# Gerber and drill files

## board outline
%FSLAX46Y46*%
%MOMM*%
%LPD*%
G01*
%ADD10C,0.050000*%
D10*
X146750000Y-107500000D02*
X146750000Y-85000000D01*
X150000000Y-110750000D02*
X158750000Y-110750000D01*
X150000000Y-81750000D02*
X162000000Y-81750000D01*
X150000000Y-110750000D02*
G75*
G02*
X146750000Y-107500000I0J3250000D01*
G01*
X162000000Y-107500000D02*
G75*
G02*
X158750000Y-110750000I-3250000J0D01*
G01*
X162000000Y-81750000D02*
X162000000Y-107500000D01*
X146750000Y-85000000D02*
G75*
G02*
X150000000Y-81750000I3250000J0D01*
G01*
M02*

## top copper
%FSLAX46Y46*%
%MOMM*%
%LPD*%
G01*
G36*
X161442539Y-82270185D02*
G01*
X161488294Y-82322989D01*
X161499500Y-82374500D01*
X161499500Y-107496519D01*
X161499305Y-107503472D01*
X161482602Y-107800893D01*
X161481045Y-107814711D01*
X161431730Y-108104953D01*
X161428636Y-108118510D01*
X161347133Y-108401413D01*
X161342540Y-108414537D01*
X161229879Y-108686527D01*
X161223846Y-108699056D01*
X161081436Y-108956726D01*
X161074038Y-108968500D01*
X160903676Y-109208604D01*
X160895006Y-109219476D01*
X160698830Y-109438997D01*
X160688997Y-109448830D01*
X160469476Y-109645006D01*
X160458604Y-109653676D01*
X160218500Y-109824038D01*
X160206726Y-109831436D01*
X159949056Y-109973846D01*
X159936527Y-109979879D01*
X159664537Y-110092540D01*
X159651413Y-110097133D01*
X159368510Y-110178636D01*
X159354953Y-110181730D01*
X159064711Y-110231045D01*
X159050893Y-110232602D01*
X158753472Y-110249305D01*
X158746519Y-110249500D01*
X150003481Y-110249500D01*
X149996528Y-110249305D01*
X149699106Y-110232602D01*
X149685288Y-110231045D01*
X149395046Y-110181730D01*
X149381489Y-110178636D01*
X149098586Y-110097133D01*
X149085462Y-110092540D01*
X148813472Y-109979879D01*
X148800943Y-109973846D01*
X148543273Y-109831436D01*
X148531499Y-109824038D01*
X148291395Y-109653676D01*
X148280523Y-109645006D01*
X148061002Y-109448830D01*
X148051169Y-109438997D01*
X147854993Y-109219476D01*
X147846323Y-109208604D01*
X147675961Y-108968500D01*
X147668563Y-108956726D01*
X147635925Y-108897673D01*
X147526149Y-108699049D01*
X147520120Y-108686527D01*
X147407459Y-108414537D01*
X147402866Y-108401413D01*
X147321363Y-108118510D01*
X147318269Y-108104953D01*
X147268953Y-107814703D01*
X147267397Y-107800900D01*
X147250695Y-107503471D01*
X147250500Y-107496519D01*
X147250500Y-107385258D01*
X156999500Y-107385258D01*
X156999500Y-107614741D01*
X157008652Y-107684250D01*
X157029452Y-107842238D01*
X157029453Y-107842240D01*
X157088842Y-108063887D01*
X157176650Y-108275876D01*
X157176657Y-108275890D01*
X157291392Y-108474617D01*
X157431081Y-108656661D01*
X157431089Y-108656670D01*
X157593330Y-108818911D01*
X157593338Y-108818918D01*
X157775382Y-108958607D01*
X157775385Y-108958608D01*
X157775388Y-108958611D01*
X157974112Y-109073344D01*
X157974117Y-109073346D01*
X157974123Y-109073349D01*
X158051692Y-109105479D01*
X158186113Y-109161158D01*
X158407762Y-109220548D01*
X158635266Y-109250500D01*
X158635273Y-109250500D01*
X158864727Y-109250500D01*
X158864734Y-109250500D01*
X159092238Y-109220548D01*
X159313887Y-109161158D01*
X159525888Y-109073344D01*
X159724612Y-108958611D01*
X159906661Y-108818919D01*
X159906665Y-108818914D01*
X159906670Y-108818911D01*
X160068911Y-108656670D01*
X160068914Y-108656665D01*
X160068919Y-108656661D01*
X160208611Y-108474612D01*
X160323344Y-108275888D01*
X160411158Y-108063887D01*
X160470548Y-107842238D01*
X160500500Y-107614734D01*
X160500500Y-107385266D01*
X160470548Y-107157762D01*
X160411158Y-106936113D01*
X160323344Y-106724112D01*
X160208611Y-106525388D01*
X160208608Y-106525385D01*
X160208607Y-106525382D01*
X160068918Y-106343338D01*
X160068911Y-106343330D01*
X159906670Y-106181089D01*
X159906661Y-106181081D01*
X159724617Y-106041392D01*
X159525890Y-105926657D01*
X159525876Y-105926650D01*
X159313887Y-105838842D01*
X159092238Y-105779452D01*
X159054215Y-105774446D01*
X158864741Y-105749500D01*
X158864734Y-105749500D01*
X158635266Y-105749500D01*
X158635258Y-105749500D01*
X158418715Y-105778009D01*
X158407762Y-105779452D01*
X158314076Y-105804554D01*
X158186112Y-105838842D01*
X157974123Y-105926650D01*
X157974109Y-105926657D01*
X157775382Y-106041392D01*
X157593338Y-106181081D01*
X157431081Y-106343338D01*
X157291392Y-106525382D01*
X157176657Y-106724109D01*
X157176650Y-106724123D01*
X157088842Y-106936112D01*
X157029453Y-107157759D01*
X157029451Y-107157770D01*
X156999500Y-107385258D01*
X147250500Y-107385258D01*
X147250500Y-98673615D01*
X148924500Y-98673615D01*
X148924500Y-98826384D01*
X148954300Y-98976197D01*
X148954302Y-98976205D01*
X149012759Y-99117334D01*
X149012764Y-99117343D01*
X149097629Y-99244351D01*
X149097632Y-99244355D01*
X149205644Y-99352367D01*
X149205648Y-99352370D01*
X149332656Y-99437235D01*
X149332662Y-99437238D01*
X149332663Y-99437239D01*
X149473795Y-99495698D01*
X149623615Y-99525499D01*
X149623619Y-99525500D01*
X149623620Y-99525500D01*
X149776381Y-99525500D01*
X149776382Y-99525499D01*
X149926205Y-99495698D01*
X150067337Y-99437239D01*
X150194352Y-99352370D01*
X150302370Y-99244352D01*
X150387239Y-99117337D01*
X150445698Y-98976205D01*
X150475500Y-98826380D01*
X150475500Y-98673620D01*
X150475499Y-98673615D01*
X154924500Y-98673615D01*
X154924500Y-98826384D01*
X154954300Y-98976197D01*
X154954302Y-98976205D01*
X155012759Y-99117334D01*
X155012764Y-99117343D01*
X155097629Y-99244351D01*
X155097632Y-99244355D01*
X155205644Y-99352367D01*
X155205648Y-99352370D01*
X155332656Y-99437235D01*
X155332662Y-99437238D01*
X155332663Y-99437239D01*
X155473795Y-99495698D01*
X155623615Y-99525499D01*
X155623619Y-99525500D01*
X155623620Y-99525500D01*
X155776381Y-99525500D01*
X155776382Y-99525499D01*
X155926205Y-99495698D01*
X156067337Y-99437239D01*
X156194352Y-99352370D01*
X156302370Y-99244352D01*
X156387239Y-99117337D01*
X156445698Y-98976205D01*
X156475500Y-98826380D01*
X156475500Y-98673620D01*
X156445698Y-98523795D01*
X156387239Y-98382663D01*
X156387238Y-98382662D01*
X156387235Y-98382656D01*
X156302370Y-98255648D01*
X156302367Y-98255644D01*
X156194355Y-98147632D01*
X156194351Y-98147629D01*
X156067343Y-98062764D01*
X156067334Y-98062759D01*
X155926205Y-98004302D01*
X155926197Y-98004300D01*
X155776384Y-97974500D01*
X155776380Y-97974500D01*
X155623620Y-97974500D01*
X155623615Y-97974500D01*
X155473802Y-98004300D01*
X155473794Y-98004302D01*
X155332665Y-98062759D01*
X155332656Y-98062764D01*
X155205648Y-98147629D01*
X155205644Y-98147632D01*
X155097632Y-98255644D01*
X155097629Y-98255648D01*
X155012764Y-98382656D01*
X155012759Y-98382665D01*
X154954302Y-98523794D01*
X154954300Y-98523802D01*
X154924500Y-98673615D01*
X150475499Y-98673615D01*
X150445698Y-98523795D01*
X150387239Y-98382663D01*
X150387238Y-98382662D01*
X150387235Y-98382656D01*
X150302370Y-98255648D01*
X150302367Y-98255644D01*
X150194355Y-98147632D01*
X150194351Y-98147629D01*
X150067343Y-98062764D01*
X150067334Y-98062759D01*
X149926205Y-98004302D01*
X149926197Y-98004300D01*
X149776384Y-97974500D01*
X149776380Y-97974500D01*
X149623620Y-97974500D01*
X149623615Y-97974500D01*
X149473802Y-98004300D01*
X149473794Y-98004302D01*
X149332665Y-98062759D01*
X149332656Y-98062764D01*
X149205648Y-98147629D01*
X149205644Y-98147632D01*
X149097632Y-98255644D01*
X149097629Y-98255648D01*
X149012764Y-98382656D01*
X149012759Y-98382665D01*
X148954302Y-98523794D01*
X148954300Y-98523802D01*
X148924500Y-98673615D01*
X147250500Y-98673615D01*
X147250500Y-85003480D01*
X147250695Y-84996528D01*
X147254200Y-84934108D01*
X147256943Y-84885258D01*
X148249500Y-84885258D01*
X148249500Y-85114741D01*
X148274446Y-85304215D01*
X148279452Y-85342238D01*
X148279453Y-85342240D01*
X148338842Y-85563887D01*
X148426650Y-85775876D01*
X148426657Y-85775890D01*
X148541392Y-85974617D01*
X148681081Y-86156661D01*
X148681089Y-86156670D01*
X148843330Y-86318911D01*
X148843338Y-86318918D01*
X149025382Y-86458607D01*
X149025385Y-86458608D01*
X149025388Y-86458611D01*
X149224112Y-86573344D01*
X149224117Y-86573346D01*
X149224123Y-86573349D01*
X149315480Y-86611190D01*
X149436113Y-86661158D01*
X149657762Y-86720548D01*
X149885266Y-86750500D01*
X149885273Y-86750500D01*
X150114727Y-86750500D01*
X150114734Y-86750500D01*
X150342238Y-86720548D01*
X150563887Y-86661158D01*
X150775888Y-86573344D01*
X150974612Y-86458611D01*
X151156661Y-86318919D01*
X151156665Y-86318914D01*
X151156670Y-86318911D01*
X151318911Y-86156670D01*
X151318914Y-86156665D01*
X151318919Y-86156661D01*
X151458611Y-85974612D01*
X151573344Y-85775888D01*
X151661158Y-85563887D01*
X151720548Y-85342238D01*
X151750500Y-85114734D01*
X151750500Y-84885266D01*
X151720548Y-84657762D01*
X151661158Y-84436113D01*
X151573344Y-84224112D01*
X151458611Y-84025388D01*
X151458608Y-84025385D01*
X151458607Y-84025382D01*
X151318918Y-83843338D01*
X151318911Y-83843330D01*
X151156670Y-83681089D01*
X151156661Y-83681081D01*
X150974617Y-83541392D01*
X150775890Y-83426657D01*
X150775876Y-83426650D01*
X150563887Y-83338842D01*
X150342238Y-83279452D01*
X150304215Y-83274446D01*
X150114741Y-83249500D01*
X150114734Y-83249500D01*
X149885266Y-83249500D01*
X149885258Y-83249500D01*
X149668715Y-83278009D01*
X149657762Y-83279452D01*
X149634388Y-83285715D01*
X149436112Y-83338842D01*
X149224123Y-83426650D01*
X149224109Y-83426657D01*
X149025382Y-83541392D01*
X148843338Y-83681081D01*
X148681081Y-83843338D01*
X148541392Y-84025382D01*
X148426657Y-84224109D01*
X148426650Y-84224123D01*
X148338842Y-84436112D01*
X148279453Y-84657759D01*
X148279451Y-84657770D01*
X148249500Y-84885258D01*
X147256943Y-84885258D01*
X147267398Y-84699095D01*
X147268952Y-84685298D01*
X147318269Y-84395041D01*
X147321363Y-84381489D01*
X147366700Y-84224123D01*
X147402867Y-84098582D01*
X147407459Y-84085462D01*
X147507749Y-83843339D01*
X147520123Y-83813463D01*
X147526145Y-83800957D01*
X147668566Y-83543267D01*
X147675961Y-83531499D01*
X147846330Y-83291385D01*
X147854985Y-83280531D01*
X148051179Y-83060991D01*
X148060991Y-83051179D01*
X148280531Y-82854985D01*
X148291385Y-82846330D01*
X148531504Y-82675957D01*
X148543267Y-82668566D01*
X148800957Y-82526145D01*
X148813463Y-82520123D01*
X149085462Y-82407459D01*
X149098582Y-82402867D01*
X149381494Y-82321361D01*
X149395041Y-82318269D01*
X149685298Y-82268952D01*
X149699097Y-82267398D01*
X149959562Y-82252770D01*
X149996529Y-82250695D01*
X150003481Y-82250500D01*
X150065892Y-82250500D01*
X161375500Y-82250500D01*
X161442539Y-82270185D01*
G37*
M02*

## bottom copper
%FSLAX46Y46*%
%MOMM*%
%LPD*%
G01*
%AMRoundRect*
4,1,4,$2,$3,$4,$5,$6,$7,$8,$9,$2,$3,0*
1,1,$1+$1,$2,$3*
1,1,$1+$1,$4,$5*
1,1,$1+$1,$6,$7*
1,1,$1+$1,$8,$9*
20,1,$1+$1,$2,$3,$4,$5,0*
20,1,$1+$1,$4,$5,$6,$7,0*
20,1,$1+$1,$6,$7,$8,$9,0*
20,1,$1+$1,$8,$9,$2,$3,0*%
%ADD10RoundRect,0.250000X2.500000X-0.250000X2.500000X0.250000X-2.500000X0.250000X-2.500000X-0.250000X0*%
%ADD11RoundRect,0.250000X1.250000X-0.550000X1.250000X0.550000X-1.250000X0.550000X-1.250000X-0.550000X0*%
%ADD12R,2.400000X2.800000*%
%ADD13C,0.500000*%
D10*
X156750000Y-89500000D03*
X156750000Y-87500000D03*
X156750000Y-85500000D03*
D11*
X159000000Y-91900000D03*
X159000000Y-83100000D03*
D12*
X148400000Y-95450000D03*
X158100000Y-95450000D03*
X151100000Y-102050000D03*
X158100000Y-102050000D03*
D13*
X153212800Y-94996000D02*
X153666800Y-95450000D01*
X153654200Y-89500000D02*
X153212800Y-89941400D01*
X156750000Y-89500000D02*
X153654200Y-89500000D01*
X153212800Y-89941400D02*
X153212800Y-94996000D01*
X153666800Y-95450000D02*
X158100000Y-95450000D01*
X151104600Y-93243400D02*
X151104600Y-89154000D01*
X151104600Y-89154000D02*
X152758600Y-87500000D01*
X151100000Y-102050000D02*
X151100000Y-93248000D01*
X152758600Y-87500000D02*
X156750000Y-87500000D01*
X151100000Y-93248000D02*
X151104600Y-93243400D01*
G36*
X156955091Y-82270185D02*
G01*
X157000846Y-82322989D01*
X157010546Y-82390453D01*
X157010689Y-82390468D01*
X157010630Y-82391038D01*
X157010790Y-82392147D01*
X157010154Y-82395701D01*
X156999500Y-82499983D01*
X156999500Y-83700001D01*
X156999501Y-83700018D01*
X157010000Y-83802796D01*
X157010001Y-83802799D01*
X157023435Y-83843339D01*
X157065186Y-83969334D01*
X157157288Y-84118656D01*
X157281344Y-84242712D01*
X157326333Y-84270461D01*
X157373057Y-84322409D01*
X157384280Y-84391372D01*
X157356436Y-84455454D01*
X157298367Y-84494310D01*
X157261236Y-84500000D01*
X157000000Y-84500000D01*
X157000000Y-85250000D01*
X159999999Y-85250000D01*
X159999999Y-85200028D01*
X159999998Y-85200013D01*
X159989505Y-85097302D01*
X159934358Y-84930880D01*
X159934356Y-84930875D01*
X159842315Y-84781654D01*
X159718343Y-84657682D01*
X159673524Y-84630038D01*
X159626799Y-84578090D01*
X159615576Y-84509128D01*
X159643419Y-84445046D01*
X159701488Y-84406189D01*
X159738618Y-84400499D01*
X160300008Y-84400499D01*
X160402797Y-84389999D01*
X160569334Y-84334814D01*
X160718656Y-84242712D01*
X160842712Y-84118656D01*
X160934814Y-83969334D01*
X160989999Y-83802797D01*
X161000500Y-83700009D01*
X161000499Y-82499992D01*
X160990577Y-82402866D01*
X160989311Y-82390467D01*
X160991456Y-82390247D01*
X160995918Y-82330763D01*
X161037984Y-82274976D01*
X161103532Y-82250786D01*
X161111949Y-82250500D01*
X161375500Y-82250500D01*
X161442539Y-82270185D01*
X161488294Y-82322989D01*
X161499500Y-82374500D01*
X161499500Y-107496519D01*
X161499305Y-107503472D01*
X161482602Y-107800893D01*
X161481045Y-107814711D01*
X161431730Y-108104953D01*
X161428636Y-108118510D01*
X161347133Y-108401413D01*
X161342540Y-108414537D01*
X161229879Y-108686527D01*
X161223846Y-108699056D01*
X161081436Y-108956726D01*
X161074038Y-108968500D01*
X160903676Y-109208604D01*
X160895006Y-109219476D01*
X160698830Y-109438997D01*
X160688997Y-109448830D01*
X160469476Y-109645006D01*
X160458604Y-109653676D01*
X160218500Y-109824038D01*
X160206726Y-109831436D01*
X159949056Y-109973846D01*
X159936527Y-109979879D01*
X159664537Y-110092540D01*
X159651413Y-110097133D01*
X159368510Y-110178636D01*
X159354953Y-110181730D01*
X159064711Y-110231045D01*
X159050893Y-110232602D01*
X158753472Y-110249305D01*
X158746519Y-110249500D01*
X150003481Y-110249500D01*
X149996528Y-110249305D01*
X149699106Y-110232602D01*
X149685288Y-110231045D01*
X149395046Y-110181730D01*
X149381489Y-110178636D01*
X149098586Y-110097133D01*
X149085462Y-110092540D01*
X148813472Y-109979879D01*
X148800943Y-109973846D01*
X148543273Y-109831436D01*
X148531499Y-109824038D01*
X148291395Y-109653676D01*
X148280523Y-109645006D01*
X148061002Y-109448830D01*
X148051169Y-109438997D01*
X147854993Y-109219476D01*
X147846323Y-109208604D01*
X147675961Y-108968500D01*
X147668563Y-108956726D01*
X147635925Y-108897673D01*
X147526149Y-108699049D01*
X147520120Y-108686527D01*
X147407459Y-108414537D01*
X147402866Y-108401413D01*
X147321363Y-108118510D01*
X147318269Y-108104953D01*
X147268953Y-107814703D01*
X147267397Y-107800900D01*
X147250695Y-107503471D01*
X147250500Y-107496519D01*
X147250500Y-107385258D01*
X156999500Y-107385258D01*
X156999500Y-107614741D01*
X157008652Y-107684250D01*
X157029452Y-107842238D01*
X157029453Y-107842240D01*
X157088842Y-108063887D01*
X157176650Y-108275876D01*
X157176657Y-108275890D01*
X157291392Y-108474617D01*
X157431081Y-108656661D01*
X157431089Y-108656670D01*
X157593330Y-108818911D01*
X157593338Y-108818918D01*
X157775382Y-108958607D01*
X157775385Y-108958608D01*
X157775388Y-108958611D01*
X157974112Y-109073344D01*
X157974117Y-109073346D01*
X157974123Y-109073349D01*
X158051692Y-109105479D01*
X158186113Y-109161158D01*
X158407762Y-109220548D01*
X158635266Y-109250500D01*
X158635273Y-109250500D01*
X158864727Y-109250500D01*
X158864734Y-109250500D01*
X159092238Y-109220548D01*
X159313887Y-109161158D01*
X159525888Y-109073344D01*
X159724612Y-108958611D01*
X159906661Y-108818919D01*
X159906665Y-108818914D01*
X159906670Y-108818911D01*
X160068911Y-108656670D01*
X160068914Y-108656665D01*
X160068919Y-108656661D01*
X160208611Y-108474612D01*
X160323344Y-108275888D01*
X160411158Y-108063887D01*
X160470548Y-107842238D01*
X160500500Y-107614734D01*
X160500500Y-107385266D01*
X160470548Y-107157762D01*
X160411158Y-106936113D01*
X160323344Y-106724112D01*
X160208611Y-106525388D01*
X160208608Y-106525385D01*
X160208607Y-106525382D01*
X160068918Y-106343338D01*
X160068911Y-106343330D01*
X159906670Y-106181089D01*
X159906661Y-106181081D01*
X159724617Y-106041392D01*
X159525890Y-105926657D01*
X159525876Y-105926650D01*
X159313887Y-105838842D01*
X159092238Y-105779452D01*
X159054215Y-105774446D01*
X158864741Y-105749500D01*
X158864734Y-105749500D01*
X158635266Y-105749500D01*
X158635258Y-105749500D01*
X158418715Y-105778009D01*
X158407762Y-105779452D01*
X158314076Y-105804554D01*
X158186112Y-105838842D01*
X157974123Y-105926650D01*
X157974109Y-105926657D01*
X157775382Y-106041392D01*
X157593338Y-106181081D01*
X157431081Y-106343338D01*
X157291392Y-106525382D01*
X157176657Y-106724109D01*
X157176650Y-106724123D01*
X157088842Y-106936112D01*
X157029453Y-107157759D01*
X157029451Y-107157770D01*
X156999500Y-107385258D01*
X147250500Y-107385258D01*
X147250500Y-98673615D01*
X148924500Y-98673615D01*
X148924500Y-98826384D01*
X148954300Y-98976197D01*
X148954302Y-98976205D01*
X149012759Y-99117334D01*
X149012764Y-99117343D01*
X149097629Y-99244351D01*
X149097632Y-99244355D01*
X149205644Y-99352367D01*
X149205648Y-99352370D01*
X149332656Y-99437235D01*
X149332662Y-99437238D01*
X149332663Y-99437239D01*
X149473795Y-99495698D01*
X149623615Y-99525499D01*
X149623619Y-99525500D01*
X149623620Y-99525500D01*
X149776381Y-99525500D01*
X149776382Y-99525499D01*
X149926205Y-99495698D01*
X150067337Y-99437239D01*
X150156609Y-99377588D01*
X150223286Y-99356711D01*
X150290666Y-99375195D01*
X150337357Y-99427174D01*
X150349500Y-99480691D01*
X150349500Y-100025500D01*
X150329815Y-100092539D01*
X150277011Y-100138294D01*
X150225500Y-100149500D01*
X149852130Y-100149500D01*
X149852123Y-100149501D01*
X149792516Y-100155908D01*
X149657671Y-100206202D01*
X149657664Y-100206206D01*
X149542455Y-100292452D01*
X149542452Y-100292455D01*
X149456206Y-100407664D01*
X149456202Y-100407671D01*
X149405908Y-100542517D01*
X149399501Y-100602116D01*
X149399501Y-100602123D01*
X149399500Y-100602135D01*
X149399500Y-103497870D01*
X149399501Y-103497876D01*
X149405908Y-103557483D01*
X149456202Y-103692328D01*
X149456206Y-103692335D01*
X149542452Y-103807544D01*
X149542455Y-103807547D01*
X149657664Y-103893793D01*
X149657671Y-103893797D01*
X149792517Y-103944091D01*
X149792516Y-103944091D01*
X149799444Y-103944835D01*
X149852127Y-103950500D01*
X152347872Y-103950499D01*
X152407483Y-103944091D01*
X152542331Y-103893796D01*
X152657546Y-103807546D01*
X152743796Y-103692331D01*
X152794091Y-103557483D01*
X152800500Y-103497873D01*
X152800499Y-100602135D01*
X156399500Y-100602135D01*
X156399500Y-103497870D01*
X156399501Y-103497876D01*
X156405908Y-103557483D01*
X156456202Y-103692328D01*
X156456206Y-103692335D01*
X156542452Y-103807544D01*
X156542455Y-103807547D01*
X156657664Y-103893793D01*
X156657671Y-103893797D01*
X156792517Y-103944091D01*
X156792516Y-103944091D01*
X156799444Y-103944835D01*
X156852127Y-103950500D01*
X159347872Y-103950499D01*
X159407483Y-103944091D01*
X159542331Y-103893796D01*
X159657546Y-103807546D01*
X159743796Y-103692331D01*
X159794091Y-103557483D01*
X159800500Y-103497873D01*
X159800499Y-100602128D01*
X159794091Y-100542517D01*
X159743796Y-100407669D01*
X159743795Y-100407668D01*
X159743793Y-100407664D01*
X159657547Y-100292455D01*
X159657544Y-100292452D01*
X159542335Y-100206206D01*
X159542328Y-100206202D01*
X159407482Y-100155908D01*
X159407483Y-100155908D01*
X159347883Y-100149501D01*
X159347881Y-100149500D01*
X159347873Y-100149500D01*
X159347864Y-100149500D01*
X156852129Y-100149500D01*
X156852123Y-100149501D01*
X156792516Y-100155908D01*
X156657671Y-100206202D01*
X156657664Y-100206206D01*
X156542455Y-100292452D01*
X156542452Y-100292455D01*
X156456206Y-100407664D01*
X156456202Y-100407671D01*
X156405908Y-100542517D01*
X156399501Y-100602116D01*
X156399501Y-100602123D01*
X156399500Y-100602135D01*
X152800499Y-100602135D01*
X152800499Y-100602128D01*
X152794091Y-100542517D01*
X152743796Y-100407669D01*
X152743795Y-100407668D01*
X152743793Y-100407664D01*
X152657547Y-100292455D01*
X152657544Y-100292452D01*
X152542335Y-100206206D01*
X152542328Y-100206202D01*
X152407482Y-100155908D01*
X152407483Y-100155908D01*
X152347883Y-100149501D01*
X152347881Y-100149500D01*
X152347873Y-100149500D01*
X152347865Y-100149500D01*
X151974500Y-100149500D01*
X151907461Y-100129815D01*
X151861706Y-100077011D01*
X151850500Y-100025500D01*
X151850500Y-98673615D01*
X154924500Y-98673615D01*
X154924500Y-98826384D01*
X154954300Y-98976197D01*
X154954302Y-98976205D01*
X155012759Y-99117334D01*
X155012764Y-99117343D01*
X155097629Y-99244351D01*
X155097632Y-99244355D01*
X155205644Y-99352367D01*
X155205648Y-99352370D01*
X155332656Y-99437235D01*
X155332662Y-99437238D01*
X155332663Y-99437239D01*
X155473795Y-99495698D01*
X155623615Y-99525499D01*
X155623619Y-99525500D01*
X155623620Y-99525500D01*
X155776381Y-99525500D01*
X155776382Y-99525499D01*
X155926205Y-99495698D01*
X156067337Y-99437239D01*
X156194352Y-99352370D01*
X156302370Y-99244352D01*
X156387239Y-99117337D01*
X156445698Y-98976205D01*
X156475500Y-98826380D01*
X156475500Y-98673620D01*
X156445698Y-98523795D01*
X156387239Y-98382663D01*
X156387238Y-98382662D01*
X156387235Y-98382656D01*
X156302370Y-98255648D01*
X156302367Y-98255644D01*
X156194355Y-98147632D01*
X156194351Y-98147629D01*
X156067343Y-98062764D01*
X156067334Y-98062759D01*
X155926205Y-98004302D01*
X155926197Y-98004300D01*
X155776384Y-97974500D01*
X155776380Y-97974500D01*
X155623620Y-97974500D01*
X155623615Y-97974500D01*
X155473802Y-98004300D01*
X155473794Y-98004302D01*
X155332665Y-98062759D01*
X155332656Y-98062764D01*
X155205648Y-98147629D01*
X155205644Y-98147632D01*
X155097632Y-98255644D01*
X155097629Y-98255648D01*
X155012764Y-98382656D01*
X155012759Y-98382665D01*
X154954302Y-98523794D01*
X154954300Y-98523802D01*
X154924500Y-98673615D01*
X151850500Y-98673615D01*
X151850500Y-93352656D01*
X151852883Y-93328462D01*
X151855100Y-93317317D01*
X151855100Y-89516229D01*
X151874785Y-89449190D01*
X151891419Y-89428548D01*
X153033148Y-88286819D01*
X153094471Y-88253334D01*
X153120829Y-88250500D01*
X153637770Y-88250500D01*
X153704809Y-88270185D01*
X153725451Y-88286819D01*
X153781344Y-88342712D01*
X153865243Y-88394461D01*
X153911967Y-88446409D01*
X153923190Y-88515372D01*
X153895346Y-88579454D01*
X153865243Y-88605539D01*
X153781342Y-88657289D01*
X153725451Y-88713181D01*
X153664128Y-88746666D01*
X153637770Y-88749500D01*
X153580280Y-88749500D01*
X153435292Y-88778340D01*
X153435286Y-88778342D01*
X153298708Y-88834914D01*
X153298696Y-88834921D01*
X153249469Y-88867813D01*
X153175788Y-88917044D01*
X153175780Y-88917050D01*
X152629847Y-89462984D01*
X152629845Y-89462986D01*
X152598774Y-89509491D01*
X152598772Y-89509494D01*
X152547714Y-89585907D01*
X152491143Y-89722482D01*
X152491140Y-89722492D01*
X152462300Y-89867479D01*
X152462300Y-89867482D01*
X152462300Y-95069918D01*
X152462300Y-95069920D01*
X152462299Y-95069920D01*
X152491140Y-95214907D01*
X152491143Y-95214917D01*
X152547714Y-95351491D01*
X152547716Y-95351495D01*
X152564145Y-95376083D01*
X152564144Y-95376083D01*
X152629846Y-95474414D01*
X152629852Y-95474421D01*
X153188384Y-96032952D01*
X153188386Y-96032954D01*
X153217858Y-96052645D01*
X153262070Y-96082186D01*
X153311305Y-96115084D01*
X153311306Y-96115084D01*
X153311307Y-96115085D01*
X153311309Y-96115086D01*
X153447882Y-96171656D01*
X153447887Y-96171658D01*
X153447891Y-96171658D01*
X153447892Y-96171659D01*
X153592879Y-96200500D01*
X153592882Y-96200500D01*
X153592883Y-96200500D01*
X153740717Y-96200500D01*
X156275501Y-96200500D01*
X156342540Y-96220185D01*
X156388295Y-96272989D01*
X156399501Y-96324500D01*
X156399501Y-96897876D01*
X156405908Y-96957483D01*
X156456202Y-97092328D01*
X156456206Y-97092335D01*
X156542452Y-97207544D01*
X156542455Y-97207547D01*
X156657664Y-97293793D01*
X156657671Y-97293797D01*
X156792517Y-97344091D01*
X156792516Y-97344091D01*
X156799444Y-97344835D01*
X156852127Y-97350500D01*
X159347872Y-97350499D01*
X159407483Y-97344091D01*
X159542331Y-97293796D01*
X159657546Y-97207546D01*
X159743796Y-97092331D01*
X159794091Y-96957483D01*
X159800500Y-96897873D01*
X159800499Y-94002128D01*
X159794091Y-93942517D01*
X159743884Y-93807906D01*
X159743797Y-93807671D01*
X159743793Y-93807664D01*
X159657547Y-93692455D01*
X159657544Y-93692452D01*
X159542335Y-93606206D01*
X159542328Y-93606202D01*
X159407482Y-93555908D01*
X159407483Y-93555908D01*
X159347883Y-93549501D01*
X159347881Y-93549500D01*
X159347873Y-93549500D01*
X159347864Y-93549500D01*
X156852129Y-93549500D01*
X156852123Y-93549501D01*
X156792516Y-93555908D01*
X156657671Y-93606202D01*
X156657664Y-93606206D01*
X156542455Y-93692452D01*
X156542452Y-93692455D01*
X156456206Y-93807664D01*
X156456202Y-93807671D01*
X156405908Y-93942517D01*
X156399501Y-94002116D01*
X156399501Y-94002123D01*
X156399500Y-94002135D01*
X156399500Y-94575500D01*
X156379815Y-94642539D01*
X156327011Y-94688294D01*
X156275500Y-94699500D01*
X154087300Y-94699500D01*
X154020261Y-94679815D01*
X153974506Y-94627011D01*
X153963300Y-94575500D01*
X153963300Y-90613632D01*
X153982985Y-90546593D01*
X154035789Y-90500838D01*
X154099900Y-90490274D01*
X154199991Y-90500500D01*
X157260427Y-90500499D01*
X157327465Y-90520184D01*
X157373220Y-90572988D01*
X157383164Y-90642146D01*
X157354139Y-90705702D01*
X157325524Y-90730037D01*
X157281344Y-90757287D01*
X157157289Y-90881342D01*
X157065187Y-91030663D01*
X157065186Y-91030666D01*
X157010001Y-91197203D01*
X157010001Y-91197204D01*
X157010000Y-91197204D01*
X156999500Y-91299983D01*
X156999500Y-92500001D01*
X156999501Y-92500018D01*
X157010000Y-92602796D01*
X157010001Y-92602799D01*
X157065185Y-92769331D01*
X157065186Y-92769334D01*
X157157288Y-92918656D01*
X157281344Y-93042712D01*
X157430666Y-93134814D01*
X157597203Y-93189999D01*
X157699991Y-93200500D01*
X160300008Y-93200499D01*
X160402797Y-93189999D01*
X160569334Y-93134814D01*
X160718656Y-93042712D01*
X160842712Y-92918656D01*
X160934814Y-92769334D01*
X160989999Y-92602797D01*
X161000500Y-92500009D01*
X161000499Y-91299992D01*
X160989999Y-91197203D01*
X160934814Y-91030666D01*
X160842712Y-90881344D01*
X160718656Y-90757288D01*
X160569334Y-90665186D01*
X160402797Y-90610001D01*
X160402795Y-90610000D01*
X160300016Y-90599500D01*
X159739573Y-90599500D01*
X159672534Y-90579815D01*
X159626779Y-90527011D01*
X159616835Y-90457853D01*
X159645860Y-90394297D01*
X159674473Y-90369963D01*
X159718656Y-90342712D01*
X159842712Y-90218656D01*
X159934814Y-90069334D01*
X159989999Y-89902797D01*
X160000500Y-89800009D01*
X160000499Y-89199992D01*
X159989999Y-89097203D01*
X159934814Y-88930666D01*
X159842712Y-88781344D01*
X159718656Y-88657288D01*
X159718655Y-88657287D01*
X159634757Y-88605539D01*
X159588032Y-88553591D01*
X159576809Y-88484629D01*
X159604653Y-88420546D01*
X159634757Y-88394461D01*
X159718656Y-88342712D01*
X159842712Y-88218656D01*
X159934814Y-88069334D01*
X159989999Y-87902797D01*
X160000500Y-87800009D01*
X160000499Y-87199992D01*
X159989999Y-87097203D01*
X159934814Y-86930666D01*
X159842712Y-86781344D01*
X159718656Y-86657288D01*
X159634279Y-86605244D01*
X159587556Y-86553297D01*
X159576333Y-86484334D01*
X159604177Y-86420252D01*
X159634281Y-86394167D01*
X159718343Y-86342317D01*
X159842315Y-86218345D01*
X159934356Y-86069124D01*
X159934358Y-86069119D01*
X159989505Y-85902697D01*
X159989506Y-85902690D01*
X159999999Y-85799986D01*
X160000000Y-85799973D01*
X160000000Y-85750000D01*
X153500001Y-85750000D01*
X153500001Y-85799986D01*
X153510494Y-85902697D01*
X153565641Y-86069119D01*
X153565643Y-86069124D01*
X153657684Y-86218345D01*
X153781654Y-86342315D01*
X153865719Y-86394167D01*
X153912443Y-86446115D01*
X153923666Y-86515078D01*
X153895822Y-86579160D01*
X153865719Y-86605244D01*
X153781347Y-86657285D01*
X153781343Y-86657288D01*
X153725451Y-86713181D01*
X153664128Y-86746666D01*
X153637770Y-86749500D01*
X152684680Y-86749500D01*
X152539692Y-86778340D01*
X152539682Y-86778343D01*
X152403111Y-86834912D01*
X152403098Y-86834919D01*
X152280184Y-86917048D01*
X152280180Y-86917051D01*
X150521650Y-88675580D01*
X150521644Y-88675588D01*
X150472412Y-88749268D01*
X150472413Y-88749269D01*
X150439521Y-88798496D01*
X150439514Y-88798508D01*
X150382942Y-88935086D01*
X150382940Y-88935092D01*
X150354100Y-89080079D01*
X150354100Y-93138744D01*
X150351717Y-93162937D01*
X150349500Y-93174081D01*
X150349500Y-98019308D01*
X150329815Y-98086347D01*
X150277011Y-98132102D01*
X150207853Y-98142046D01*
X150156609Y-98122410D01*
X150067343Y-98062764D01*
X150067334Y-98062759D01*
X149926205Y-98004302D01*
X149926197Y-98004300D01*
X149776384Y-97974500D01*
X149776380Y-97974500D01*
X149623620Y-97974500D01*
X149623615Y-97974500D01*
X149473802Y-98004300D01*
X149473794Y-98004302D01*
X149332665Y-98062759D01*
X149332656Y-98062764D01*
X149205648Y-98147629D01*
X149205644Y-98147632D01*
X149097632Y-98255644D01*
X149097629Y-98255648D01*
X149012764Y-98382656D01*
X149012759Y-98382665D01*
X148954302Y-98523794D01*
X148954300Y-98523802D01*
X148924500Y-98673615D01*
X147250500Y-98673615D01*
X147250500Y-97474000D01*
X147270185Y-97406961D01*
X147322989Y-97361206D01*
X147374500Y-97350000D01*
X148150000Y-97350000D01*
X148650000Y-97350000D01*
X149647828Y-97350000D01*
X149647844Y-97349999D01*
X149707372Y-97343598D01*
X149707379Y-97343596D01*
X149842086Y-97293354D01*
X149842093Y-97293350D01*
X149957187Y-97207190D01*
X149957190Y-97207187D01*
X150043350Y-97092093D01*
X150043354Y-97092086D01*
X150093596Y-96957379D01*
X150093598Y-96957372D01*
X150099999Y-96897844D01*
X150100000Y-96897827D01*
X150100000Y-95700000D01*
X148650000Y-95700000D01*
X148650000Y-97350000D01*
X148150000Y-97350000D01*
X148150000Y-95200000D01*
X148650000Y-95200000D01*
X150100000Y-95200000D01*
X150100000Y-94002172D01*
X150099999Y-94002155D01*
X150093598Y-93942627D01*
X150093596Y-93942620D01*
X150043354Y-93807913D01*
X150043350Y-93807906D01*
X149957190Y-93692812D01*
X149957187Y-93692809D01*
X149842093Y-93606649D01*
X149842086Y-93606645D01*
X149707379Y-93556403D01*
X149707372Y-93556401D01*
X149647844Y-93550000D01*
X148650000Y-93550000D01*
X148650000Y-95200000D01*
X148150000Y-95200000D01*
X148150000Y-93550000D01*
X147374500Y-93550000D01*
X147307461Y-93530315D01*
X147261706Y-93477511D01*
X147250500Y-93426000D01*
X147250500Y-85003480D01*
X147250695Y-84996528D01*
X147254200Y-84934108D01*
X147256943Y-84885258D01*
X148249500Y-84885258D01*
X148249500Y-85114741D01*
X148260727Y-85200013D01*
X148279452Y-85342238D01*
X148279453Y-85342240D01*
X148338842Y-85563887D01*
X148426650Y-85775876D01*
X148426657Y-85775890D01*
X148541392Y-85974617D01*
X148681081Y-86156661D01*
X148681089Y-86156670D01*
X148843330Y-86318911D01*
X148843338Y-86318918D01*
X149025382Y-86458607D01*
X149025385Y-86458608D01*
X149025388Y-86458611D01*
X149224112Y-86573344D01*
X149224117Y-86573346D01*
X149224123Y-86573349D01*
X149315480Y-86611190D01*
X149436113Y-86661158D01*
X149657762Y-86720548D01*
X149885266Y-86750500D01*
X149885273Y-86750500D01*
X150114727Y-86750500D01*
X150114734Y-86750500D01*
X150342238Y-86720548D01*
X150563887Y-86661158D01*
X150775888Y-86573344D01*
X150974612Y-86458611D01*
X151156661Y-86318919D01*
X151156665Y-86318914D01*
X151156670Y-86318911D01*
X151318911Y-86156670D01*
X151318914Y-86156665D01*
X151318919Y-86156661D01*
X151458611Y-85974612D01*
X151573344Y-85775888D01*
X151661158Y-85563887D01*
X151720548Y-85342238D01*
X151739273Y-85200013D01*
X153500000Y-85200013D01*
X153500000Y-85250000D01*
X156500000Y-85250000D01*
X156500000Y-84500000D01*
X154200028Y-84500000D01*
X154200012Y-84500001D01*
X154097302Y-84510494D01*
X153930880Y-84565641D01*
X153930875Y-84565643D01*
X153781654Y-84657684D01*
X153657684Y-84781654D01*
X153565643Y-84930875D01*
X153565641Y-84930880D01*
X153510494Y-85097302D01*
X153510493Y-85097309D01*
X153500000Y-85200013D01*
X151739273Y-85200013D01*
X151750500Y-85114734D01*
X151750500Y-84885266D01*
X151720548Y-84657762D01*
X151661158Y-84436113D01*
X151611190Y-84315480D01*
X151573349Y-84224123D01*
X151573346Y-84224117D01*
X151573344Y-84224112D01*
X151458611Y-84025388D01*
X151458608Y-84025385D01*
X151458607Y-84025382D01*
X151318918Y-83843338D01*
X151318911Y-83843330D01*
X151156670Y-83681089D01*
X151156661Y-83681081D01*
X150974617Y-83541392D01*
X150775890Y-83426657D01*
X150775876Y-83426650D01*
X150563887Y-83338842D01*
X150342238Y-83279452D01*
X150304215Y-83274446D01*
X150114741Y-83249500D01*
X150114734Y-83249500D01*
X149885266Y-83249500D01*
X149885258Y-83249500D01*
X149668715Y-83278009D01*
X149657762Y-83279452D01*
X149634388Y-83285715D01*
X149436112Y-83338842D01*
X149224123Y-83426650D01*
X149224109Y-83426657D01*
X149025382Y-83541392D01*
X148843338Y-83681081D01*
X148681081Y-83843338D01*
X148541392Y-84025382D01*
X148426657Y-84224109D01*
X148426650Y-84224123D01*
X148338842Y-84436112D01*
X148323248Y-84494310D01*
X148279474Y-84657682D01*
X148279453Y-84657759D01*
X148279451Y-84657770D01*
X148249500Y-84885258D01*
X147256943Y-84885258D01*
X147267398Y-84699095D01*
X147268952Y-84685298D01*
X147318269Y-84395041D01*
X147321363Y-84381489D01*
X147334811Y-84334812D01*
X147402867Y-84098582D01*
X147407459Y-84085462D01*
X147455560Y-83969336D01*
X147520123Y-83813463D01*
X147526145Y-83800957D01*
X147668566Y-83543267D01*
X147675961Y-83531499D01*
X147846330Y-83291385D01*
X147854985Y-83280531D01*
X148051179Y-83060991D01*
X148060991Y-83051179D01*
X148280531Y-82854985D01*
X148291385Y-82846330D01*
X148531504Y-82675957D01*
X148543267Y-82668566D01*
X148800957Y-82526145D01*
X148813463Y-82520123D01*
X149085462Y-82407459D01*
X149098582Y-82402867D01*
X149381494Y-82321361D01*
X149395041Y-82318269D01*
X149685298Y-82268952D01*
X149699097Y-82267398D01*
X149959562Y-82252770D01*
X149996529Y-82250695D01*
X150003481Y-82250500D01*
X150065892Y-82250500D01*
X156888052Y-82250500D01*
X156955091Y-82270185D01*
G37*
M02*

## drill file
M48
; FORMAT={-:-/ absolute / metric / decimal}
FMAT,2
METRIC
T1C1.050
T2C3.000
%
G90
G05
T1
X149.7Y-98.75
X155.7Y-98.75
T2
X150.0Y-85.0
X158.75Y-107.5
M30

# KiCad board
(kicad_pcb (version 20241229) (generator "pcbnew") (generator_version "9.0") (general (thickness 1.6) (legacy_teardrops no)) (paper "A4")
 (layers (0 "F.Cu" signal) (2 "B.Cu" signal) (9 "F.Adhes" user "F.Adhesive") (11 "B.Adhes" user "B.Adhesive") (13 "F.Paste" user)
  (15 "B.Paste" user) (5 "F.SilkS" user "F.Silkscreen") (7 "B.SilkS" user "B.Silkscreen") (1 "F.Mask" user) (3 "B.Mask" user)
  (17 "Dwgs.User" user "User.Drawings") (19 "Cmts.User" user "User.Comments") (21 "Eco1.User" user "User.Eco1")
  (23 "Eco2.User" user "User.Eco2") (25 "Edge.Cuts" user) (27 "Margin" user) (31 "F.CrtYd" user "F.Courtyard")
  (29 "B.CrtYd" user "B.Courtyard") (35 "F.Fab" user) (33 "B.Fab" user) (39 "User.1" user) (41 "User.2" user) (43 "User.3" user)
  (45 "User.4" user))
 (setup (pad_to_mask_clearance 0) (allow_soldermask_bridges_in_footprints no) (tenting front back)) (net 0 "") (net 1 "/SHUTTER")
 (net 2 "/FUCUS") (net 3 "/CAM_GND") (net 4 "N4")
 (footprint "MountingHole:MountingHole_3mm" (layer "F.Cu") (at 158.75 107.5)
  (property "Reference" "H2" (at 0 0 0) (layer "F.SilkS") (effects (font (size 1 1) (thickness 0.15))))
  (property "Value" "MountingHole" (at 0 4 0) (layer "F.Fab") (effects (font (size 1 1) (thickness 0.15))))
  (pad "" np_thru_hole circle (at 0 0) (size 3 3) (drill 3) (layers "*.Cu" "*.Mask")))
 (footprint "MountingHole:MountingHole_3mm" (layer "F.Cu") (at 150 85)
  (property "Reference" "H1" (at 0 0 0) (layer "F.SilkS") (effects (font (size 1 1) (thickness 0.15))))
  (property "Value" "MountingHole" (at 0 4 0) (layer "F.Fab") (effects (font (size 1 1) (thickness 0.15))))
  (pad "" np_thru_hole circle (at 0 0) (size 3 3) (drill 3) (layers "*.Cu" "*.Mask")))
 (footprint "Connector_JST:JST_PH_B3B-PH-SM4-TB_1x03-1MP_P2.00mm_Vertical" (layer "B.Cu") (at 157.25 87.5 90)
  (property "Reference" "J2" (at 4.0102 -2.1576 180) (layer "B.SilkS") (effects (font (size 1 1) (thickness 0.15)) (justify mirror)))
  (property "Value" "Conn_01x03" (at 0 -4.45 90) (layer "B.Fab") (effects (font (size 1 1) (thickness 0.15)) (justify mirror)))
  (pad "1" smd roundrect (at -2 -0.5 90) (size 1 5.5) (layers "B.Cu" "B.Mask" "B.Paste") (roundrect_rratio 0.25) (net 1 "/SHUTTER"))
  (pad "2" smd roundrect (at 0 -0.5 90) (size 1 5.5) (layers "B.Cu" "B.Mask" "B.Paste") (roundrect_rratio 0.25) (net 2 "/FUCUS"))
  (pad "3" smd roundrect (at 2 -0.5 90) (size 1 5.5) (layers "B.Cu" "B.Mask" "B.Paste") (roundrect_rratio 0.25) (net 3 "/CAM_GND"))
  (pad "MP" smd roundrect (at -4.4 1.75 90) (size 1.6 3) (layers "B.Cu" "B.Mask" "B.Paste") (roundrect_rratio 0.15625))
  (pad "MP" smd roundrect (at 4.4 1.75 90) (size 1.6 3) (layers "B.Cu" "B.Mask" "B.Paste") (roundrect_rratio 0.15625)))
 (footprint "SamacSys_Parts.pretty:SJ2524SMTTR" (layer "B.Cu") (at 152.25 98.75)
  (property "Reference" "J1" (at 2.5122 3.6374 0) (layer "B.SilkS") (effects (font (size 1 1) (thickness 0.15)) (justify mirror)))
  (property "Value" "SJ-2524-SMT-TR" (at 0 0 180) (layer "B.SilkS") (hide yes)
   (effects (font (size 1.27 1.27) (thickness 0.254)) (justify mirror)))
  (pad "" np_thru_hole circle (at -2.55 0) (size 1.05 1.05) (drill 1.05) (layers "*.Cu" "*.Mask"))
  (pad "" np_thru_hole circle (at 3.45 0) (size 1.05 1.05) (drill 1.05) (layers "*.Cu" "*.Mask"))
  (pad "1" smd rect (at -3.85 -3.3) (size 2.4 2.8) (layers "B.Cu" "B.Mask" "B.Paste") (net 3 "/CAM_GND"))
  (pad "2" smd rect (at 5.85 -3.3) (size 2.4 2.8) (layers "B.Cu" "B.Mask" "B.Paste") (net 1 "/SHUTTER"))
  (pad "3" smd rect (at -1.15 3.3) (size 2.4 2.8) (layers "B.Cu" "B.Mask" "B.Paste") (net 2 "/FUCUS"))
  (pad "4" smd rect (at 5.85 3.3) (size 2.4 2.8) (layers "B.Cu" "B.Mask" "B.Paste") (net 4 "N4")))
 (gr_line (start 146.75 107.5) (end 146.75 85) (stroke (width 0.05) (type default)) (layer "Edge.Cuts"))
 (gr_line (start 150 110.75) (end 158.75 110.75) (stroke (width 0.05) (type default)) (layer "Edge.Cuts"))
 (gr_line (start 150 81.75) (end 162 81.75) (stroke (width 0.05) (type solid)) (layer "Edge.Cuts"))
 (gr_arc (start 150 110.75) (mid 147.701903 109.798097) (end 146.75 107.5) (stroke (width 0.05) (type solid)) (layer "Edge.Cuts"))
 (gr_arc (start 162 107.5) (mid 161.048097 109.798097) (end 158.75 110.75) (stroke (width 0.05) (type solid)) (layer "Edge.Cuts"))
 (gr_line (start 162 81.75) (end 162 107.5) (stroke (width 0.05) (type default)) (layer "Edge.Cuts"))
 (gr_arc (start 146.75 85) (mid 147.701903 82.701903) (end 150 81.75) (stroke (width 0.05) (type solid)) (layer "Edge.Cuts"))
 (segment (start 153.2128 94.996) (end 153.6668 95.45) (width 0.5) (layer "B.Cu") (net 1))
 (segment (start 153.6542 89.5) (end 153.2128 89.9414) (width 0.5) (layer "B.Cu") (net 1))
 (segment (start 156.75 89.5) (end 153.6542 89.5) (width 0.5) (layer "B.Cu") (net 1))
 (segment (start 153.2128 89.9414) (end 153.2128 94.996) (width 0.5) (layer "B.Cu") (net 1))
 (segment (start 153.6668 95.45) (end 158.1 95.45) (width 0.5) (layer "B.Cu") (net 1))
 (segment (start 151.1046 93.2434) (end 151.1046 89.154) (width 0.5) (layer "B.Cu") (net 2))
 (segment (start 151.1046 89.154) (end 152.7586 87.5) (width 0.5) (layer "B.Cu") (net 2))
 (segment (start 151.1 102.05) (end 151.1 93.248) (width 0.5) (layer "B.Cu") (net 2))
 (segment (start 152.7586 87.5) (end 156.75 87.5) (width 0.5) (layer "B.Cu") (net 2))
 (segment (start 151.1 93.248) (end 151.1046 93.2434) (width 0.5) (layer "B.Cu") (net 2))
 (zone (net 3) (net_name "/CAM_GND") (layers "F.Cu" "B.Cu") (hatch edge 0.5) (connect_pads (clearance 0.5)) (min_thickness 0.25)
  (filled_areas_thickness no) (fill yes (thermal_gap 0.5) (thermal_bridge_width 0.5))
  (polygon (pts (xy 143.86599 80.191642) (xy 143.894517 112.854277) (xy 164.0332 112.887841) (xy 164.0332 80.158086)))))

